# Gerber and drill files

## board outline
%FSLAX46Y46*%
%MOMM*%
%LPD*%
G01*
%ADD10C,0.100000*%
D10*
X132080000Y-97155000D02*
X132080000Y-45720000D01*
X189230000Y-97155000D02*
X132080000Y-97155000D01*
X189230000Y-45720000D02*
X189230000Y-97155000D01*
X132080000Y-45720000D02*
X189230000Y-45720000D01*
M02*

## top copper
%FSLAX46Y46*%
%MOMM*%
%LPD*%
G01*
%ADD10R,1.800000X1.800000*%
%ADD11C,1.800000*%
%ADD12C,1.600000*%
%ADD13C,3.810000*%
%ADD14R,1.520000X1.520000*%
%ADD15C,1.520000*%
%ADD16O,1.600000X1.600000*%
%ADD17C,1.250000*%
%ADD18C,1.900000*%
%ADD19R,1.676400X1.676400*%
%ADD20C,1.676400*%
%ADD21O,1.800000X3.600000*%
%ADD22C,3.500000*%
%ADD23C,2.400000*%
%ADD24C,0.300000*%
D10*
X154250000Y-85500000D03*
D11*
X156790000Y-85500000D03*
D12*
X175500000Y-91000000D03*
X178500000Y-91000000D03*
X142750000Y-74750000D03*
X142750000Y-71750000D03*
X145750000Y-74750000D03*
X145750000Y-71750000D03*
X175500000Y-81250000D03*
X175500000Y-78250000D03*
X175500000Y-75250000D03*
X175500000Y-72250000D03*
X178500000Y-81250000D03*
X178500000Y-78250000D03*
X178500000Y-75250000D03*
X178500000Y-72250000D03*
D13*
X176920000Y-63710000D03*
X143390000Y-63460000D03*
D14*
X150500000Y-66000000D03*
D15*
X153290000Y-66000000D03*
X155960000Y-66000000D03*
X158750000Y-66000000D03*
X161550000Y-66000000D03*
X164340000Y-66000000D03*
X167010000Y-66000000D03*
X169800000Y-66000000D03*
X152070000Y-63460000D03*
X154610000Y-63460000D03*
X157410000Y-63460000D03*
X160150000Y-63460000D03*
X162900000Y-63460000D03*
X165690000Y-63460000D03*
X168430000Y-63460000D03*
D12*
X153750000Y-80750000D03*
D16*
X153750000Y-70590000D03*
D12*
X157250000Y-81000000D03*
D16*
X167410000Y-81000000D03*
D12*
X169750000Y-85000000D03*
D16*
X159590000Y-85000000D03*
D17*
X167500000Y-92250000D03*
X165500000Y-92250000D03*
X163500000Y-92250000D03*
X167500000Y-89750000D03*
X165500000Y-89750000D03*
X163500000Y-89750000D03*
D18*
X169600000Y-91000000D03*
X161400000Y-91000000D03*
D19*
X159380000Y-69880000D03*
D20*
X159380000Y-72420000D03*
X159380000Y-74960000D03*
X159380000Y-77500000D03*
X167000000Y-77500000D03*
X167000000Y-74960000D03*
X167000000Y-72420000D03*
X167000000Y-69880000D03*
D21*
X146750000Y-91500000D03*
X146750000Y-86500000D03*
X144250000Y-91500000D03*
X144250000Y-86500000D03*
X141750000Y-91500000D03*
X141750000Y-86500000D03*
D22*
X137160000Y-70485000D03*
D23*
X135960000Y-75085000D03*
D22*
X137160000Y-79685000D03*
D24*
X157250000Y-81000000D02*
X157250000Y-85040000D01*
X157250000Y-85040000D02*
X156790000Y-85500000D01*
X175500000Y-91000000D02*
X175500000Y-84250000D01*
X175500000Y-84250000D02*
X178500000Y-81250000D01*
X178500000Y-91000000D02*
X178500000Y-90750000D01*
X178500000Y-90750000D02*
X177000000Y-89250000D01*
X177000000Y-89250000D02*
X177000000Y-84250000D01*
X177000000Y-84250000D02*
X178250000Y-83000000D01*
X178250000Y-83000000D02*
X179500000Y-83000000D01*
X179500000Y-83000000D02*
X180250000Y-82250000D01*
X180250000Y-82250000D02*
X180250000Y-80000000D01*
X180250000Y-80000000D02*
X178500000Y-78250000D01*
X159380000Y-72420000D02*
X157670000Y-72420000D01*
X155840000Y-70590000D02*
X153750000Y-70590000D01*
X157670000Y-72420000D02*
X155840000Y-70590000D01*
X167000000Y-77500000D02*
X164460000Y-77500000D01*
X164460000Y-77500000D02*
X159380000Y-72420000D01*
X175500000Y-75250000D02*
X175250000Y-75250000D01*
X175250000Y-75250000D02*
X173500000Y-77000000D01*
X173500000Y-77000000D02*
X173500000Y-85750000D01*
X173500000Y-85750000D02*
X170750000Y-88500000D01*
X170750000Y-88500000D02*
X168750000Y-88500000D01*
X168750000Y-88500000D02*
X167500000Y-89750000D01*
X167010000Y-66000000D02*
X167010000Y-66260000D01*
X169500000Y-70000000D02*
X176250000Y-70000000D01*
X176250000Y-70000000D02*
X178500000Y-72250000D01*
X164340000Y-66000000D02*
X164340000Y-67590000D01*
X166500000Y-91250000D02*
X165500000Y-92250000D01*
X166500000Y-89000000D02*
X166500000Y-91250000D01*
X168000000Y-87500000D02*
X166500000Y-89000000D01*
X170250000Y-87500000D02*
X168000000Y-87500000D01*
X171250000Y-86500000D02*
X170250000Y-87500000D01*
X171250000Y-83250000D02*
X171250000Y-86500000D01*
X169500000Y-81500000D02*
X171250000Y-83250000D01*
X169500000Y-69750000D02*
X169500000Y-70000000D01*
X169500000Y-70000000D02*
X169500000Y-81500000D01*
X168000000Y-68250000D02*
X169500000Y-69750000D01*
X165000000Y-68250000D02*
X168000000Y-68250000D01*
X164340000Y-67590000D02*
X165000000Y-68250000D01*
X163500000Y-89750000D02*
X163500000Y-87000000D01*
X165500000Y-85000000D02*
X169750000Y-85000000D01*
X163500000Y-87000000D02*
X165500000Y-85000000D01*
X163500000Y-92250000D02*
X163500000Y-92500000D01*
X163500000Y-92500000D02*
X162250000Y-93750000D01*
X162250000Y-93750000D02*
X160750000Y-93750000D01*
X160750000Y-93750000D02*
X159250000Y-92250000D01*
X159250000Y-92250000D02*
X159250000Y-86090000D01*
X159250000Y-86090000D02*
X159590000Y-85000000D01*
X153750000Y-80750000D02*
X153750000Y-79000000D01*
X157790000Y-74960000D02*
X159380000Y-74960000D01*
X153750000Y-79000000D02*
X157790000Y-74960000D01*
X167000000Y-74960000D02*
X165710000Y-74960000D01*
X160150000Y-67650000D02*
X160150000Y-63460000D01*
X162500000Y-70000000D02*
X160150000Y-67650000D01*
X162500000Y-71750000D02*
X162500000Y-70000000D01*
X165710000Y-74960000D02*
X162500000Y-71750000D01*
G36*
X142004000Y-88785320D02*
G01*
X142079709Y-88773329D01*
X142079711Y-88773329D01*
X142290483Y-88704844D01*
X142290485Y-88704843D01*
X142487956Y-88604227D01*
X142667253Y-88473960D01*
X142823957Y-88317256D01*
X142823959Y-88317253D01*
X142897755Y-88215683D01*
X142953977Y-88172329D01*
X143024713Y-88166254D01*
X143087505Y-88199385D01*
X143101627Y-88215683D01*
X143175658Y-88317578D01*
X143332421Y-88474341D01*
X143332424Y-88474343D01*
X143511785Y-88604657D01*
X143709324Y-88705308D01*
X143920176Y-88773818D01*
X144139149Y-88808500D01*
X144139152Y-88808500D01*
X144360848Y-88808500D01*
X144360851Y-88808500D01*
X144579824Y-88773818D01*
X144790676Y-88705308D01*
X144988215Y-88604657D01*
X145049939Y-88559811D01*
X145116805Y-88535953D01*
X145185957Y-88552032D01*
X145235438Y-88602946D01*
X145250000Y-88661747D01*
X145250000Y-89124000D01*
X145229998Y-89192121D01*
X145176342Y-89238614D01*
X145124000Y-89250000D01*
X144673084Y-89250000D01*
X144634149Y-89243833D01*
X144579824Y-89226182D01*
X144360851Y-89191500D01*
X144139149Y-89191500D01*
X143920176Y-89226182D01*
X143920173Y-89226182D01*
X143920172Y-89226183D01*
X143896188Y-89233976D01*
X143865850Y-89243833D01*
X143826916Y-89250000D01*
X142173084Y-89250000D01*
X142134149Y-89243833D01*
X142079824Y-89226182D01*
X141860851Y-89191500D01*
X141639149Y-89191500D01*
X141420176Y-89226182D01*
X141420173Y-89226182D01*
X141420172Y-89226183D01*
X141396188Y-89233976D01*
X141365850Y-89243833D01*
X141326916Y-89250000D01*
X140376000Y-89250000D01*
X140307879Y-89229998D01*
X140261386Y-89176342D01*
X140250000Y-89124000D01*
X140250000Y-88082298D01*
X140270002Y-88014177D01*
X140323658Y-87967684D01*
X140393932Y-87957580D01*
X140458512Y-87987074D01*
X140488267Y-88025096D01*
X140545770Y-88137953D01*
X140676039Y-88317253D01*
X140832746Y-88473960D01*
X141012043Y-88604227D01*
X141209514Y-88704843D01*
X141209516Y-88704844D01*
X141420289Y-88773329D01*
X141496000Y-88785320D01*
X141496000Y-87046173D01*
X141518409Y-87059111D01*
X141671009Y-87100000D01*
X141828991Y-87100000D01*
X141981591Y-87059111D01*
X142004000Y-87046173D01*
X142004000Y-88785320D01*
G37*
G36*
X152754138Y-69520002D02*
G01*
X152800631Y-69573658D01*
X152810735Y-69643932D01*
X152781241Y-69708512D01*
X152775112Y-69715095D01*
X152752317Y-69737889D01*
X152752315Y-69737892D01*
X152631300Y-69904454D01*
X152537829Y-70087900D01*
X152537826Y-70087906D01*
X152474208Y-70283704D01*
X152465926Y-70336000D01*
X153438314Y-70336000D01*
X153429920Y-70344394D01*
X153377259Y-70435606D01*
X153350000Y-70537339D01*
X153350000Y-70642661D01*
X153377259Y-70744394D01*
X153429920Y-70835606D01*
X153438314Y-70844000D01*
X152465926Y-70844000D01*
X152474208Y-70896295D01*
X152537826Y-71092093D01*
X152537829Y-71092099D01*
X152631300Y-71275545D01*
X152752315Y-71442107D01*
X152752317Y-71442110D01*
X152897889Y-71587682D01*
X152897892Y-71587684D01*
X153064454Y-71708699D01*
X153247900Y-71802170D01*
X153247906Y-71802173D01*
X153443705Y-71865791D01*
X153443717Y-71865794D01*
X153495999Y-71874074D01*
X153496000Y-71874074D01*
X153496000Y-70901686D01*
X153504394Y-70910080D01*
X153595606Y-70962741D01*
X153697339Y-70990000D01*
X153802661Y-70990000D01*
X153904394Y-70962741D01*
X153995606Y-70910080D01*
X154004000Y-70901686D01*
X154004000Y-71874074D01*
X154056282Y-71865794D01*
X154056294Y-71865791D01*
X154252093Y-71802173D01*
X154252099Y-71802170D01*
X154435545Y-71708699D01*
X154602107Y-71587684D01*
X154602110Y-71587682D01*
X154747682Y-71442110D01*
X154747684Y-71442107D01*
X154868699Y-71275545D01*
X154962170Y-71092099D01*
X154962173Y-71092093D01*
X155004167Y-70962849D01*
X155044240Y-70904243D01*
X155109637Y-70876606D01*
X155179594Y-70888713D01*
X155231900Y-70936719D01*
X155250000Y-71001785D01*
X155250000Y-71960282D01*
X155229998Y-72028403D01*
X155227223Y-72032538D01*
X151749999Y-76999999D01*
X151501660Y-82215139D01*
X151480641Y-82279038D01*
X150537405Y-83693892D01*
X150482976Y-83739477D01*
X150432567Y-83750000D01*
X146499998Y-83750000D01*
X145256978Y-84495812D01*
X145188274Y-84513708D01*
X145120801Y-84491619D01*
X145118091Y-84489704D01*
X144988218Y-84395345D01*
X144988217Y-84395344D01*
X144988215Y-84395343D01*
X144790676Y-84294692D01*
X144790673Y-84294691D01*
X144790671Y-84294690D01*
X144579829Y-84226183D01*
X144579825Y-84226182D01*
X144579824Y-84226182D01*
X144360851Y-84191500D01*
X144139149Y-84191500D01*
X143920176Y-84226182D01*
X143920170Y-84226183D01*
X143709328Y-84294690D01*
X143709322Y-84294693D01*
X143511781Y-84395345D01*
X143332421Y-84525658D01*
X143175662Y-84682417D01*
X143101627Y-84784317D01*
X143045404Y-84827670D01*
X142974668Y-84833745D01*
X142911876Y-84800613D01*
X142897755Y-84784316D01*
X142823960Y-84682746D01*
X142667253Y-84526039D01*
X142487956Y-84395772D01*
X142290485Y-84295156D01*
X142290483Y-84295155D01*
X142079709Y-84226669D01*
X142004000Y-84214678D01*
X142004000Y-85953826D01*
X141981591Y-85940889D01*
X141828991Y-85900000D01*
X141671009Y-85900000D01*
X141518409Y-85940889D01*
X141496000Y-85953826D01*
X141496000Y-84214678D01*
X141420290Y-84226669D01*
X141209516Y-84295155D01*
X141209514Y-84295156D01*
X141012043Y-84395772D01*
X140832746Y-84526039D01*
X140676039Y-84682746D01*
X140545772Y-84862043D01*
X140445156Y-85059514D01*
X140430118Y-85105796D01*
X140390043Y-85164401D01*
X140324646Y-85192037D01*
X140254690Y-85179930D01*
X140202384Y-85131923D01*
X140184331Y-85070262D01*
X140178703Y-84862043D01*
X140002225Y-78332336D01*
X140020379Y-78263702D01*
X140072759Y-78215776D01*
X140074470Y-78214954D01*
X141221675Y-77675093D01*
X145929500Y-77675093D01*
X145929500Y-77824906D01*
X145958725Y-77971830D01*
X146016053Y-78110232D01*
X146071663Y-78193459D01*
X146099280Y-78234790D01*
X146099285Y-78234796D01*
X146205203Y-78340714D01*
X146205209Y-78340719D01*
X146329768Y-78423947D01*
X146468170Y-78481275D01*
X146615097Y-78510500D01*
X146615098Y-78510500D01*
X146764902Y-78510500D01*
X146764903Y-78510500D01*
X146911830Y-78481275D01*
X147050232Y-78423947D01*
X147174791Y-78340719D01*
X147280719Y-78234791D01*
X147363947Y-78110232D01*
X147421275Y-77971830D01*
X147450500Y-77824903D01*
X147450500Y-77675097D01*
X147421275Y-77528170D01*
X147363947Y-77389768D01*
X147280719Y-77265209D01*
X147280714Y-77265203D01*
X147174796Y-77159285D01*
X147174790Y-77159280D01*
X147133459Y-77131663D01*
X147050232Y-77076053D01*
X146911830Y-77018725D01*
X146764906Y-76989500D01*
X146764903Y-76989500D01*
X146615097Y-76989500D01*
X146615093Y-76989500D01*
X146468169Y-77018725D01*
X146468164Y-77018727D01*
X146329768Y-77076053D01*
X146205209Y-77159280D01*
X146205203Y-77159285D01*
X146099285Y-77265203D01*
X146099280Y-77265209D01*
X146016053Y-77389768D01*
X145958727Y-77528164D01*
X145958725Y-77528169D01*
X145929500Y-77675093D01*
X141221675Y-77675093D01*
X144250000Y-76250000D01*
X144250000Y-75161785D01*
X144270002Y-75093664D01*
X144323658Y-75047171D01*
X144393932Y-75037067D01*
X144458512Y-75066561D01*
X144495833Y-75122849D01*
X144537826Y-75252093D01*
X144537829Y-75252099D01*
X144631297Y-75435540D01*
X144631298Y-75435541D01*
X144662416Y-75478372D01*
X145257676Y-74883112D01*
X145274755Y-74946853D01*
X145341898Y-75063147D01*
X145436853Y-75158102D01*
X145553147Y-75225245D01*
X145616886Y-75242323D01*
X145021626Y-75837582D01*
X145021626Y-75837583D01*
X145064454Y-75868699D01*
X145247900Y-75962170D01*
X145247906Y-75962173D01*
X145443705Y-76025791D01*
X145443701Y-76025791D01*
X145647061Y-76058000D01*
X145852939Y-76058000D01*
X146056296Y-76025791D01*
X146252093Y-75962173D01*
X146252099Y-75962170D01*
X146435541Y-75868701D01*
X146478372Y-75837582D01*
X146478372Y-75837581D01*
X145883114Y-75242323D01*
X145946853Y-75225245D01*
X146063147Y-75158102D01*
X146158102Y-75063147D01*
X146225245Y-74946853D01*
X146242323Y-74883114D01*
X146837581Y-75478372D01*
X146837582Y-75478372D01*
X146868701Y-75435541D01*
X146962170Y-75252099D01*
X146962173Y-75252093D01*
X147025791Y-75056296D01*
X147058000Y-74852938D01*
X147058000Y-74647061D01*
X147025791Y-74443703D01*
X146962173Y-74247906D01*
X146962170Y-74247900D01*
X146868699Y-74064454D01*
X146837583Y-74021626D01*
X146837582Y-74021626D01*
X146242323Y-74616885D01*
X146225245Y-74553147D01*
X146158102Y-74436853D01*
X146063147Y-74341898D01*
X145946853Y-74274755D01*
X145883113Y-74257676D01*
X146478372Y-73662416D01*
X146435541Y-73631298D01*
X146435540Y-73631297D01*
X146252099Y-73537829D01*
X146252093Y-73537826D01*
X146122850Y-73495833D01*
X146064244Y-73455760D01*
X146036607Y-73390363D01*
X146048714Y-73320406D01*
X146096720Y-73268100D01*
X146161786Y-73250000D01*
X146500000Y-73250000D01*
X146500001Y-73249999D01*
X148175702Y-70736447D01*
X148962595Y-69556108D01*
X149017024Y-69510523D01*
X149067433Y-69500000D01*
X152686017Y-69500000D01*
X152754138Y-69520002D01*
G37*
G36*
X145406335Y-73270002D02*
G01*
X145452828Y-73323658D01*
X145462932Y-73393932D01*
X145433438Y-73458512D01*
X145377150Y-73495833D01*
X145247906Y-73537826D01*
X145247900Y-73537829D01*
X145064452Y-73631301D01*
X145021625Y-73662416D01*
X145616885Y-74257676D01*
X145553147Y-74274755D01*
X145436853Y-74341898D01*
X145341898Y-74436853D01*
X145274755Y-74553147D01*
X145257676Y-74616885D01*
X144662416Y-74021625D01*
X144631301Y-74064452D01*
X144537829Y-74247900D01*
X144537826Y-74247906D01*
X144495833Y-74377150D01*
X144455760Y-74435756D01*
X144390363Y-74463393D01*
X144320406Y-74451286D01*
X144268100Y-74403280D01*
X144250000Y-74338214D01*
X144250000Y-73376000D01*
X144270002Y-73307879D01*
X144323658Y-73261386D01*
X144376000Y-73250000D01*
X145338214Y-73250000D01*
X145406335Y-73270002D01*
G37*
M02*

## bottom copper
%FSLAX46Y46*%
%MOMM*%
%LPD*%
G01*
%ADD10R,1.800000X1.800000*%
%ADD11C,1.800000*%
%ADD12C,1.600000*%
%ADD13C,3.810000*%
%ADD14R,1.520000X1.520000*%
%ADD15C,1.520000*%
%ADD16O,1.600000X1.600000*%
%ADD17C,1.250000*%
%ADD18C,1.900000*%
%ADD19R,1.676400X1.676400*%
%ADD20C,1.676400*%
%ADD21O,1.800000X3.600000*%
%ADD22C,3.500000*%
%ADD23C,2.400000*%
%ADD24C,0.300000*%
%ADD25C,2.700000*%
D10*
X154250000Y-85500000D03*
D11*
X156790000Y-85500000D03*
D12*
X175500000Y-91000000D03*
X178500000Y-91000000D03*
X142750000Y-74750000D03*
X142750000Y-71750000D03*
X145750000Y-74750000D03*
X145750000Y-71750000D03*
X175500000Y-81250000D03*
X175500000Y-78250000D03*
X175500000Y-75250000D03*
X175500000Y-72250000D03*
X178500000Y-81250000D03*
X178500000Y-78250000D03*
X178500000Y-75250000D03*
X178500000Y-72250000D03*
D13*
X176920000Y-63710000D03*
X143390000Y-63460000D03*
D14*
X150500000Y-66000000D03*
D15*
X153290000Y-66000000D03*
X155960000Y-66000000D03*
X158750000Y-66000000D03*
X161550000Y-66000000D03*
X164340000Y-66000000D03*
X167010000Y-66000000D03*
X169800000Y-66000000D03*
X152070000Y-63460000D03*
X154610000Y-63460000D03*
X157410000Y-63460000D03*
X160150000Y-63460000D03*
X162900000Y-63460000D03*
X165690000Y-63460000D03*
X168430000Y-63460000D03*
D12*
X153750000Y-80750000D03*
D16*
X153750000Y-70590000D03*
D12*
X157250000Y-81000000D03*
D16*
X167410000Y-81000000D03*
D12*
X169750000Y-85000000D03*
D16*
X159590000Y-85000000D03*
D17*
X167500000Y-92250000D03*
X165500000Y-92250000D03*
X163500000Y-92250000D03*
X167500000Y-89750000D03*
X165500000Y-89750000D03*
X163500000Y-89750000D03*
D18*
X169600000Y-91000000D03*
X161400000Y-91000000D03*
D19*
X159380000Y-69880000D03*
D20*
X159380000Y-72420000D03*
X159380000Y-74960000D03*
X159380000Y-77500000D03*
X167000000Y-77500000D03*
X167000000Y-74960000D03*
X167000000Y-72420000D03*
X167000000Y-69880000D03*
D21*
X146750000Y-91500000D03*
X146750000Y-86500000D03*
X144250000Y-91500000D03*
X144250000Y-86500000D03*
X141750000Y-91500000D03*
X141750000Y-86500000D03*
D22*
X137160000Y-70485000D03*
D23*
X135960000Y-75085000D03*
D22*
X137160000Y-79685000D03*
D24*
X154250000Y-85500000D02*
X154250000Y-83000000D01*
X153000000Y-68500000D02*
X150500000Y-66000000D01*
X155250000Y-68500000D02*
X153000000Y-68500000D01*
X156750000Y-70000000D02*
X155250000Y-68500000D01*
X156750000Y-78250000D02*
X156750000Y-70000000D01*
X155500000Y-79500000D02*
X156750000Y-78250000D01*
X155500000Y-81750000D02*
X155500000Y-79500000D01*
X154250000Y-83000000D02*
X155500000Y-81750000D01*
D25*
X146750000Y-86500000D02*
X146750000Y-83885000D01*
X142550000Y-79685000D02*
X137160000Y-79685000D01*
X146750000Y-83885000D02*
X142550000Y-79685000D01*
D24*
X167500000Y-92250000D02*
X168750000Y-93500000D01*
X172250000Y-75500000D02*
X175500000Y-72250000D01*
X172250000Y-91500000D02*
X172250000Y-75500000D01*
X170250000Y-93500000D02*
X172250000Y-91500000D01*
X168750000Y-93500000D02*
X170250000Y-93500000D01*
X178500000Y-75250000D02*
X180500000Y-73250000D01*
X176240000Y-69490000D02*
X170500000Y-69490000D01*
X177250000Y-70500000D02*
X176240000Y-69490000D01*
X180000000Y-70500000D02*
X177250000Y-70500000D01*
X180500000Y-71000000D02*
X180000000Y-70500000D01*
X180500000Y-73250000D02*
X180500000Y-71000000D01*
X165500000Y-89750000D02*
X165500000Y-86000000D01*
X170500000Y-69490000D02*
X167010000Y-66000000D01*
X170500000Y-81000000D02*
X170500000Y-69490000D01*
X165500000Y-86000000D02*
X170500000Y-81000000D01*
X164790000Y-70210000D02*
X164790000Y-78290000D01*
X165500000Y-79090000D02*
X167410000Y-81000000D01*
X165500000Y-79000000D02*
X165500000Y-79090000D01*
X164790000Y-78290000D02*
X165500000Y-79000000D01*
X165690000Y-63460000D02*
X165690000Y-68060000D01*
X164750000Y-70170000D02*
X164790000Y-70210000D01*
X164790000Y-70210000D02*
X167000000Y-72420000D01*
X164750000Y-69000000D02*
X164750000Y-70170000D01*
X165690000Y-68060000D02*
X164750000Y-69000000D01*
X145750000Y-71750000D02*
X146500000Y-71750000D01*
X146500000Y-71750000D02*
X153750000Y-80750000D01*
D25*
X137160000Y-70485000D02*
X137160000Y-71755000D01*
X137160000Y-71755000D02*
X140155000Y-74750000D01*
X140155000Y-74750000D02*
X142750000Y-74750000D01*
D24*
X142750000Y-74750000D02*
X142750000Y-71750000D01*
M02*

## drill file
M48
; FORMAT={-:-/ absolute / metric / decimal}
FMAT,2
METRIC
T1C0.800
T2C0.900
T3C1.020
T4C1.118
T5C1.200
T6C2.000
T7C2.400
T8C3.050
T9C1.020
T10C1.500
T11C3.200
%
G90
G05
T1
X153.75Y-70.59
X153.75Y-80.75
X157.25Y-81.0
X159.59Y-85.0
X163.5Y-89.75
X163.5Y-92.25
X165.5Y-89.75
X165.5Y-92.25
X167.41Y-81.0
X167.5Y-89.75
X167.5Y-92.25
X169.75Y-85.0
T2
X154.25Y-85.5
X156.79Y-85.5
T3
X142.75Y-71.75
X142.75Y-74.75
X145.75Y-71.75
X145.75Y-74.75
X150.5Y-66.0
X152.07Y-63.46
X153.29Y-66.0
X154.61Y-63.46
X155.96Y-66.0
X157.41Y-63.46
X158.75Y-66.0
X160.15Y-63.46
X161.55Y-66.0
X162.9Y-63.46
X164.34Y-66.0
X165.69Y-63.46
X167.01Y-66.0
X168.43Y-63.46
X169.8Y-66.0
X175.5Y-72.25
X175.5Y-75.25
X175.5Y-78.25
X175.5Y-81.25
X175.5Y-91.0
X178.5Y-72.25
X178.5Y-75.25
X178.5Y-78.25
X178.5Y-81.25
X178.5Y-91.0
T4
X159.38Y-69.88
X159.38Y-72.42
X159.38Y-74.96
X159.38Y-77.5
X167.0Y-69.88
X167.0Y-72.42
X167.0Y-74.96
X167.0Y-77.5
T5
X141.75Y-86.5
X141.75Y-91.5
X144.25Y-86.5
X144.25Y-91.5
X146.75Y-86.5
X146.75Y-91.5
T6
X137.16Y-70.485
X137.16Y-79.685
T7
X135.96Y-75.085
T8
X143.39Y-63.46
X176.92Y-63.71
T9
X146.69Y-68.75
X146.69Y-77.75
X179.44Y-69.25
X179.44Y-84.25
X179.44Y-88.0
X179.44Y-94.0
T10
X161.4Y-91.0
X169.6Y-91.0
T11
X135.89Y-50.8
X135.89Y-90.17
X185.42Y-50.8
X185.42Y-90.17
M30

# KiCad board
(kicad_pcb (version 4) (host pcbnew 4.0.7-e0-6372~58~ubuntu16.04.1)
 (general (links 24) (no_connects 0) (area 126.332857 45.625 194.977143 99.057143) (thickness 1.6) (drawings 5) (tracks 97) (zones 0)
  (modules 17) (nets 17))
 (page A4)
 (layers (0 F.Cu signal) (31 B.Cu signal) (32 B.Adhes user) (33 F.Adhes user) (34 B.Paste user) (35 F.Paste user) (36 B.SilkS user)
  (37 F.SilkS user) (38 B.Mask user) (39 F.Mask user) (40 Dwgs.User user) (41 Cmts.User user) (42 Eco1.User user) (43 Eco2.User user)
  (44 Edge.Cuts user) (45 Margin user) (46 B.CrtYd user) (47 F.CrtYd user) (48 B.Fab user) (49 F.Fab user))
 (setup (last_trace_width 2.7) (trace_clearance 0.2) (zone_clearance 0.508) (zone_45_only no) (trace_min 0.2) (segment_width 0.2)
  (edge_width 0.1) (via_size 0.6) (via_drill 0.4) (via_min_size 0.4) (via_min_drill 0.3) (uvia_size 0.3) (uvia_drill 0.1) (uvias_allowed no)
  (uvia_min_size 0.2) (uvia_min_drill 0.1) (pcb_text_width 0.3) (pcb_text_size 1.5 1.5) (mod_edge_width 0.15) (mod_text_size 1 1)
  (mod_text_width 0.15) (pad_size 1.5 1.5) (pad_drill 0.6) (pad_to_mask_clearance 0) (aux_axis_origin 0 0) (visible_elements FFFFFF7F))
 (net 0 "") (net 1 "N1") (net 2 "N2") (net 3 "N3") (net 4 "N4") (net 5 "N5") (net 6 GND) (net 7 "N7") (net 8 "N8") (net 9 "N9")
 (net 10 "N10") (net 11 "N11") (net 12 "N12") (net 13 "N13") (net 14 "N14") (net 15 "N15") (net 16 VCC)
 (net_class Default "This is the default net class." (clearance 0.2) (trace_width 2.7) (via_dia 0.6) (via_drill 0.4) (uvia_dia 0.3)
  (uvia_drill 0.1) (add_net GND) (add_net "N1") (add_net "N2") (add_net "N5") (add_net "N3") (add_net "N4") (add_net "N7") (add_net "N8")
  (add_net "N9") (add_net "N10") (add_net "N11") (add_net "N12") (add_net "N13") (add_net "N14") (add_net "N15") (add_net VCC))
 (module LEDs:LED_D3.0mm (layer F.Cu) (at 154.25 85.5)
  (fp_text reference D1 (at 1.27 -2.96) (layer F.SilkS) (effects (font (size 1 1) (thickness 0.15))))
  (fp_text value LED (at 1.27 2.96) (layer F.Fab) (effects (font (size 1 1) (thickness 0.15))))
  (pad 1 thru_hole rect (at 0 0) (size 1.8 1.8) (drill 0.9) (layers *.Cu *.Mask) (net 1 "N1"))
  (pad 2 thru_hole circle (at 2.54 0) (size 1.8 1.8) (drill 0.9) (layers *.Cu *.Mask) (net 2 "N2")))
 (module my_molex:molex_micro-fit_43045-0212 (layer F.Cu) (at 178.5 91 270)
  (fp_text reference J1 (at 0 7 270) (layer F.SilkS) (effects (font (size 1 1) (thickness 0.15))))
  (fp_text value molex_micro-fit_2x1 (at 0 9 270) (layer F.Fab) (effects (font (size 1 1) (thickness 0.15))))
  (pad 1 thru_hole circle (at 0 3 270) (size 1.6 1.6) (drill 1.02) (layers *.Cu *.Mask) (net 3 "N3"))
  (pad 2 thru_hole circle (at 0 0 270) (size 1.6 1.6) (drill 1.02) (layers *.Cu *.Mask) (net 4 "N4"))
  (pad "" np_thru_hole circle (at -3 -0.94 270) (size 1.02 1.02) (drill 1.02) (layers *.Cu *.Mask))
  (pad "" np_thru_hole circle (at 3 -0.94 270) (size 1.02 1.02) (drill 1.02) (layers *.Cu *.Mask)))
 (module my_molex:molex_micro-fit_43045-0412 (layer F.Cu) (at 145.75 73.25 270)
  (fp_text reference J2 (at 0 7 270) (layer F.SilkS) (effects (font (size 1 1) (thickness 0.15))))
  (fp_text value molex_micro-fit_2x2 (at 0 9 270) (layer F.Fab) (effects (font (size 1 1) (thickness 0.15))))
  (pad 1 thru_hole circle (at 1.5 3 270) (size 1.6 1.6) (drill 1.02) (layers *.Cu *.Mask) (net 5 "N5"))
  (pad 2 thru_hole circle (at -1.5 3 270) (size 1.6 1.6) (drill 1.02) (layers *.Cu *.Mask) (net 5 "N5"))
  (pad 3 thru_hole circle (at 1.5 0 270) (size 1.6 1.6) (drill 1.02) (layers *.Cu *.Mask) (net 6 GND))
  (pad 4 thru_hole circle (at -1.5 0 270) (size 1.6 1.6) (drill 1.02) (layers *.Cu *.Mask) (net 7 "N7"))
  (pad "" np_thru_hole circle (at -4.5 -0.94 270) (size 1.02 1.02) (drill 1.02) (layers *.Cu *.Mask))
  (pad "" np_thru_hole circle (at 4.5 -0.94 270) (size 1.02 1.02) (drill 1.02) (layers *.Cu *.Mask)))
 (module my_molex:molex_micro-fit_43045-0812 (layer F.Cu) (at 178.5 76.75 270)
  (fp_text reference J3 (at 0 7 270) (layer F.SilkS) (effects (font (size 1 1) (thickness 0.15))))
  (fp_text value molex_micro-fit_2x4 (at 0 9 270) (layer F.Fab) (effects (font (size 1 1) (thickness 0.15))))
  (pad 1 thru_hole circle (at 4.5 3 270) (size 1.6 1.6) (drill 1.02) (layers *.Cu *.Mask))
  (pad 2 thru_hole circle (at 1.5 3 270) (size 1.6 1.6) (drill 1.02) (layers *.Cu *.Mask))
  (pad 3 thru_hole circle (at -1.5 3 270) (size 1.6 1.6) (drill 1.02) (layers *.Cu *.Mask) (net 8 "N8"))
  (pad 4 thru_hole circle (at -4.5 3 270) (size 1.6 1.6) (drill 1.02) (layers *.Cu *.Mask) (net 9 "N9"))
  (pad 5 thru_hole circle (at 4.5 0 270) (size 1.6 1.6) (drill 1.02) (layers *.Cu *.Mask) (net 3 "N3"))
  (pad 6 thru_hole circle (at 1.5 0 270) (size 1.6 1.6) (drill 1.02) (layers *.Cu *.Mask) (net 4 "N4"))
  (pad 7 thru_hole circle (at -1.5 0 270) (size 1.6 1.6) (drill 1.02) (layers *.Cu *.Mask) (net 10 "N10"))
  (pad 8 thru_hole circle (at -4.5 0 270) (size 1.6 1.6) (drill 1.02) (layers *.Cu *.Mask) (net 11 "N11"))
  (pad "" np_thru_hole circle (at -7.5 -0.94 270) (size 1.02 1.02) (drill 1.02) (layers *.Cu *.Mask))
  (pad "" np_thru_hole circle (at 7.5 -0.94 270) (size 1.02 1.02) (drill 1.02) (layers *.Cu *.Mask)))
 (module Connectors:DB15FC (layer F.Cu) (at 150.5 66)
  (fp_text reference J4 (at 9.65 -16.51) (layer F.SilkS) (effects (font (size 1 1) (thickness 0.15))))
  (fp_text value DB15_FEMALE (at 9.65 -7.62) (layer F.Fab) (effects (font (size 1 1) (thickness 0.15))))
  (pad "" thru_hole circle (at 26.42 -2.29) (size 3.81 3.81) (drill 3.05) (layers *.Cu *.Mask))
  (pad "" thru_hole circle (at -7.11 -2.54) (size 3.81 3.81) (drill 3.05) (layers *.Cu *.Mask))
  (pad 1 thru_hole rect (at 0 0) (size 1.52 1.52) (drill 1.02) (layers *.Cu *.Mask) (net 1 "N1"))
  (pad 2 thru_hole circle (at 2.79 0) (size 1.52 1.52) (drill 1.02) (layers *.Cu *.Mask))
  (pad 3 thru_hole circle (at 5.46 0) (size 1.52 1.52) (drill 1.02) (layers *.Cu *.Mask))
  (pad 4 thru_hole circle (at 8.25 0) (size 1.52 1.52) (drill 1.02) (layers *.Cu *.Mask))
  (pad 5 thru_hole circle (at 11.05 0) (size 1.52 1.52) (drill 1.02) (layers *.Cu *.Mask))
  (pad 6 thru_hole circle (at 13.84 0) (size 1.52 1.52) (drill 1.02) (layers *.Cu *.Mask) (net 11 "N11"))
  (pad 7 thru_hole circle (at 16.51 0) (size 1.52 1.52) (drill 1.02) (layers *.Cu *.Mask) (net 10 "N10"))
  (pad 8 thru_hole circle (at 19.3 0) (size 1.52 1.52) (drill 1.02) (layers *.Cu *.Mask))
  (pad 9 thru_hole circle (at 1.57 -2.54) (size 1.52 1.52) (drill 1.02) (layers *.Cu *.Mask))
  (pad 10 thru_hole circle (at 4.11 -2.54) (size 1.52 1.52) (drill 1.02) (layers *.Cu *.Mask))
  (pad 11 thru_hole circle (at 6.91 -2.54) (size 1.52 1.52) (drill 1.02) (layers *.Cu *.Mask))
  (pad 12 thru_hole circle (at 9.65 -2.54) (size 1.52 1.52) (drill 1.02) (layers *.Cu *.Mask) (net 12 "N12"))
  (pad 13 thru_hole circle (at 12.4 -2.54) (size 1.52 1.52) (drill 1.02) (layers *.Cu *.Mask))
  (pad 14 thru_hole circle (at 15.19 -2.54) (size 1.52 1.52) (drill 1.02) (layers *.Cu *.Mask) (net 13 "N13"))
  (pad 15 thru_hole circle (at 17.93 -2.54) (size 1.52 1.52) (drill 1.02) (layers *.Cu *.Mask)))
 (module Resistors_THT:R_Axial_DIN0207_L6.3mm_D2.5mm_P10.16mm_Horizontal (layer F.Cu) (at 153.75 80.75 90)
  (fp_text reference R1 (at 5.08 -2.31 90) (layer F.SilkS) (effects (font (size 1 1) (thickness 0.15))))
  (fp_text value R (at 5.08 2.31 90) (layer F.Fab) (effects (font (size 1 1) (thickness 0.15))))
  (pad 1 thru_hole circle (at 0 0 90) (size 1.6 1.6) (drill 0.8) (layers *.Cu *.Mask) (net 7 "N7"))
  (pad 2 thru_hole oval (at 10.16 0 90) (size 1.6 1.6) (drill 0.8) (layers *.Cu *.Mask) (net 6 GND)))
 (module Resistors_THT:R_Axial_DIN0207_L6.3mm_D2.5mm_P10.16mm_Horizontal (layer F.Cu) (at 157.25 81)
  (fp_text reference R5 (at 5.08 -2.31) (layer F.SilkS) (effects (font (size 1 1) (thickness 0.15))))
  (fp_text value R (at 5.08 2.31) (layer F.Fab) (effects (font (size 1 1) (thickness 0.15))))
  (pad 1 thru_hole circle (at 0 0) (size 1.6 1.6) (drill 0.8) (layers *.Cu *.Mask) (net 2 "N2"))
  (pad 2 thru_hole oval (at 10.16 0) (size 1.6 1.6) (drill 0.8) (layers *.Cu *.Mask) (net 13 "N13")))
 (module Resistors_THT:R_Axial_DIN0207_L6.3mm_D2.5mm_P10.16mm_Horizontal (layer F.Cu) (at 169.75 85 180)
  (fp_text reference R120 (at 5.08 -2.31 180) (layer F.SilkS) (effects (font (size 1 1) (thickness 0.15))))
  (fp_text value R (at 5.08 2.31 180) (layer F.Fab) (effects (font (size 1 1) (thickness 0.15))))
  (pad 1 thru_hole circle (at 0 0 180) (size 1.6 1.6) (drill 0.8) (layers *.Cu *.Mask) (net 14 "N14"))
  (pad 2 thru_hole oval (at 10.16 0 180) (size 1.6 1.6) (drill 0.8) (layers *.Cu *.Mask) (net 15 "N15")))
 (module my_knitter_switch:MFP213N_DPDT (layer F.Cu) (at 165.5 91 180)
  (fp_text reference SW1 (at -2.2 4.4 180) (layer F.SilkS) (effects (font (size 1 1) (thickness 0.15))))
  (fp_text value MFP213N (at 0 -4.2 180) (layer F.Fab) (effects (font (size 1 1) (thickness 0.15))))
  (pad 1 thru_hole circle (at -2 -1.25 180) (size 1.25 1.25) (drill 0.8) (layers *.Cu *.Mask) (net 9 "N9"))
  (pad 2 thru_hole circle (at 0 -1.25 180) (size 1.25 1.25) (drill 0.8) (layers *.Cu *.Mask) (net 11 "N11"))
  (pad 3 thru_hole circle (at 2 -1.25 180) (size 1.25 1.25) (drill 0.8) (layers *.Cu *.Mask) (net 15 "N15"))
  (pad 4 thru_hole circle (at -2 1.25 180) (size 1.25 1.25) (drill 0.8) (layers *.Cu *.Mask) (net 8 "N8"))
  (pad 5 thru_hole circle (at 0 1.25 180) (size 1.25 1.25) (drill 0.8) (layers *.Cu *.Mask) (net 10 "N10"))
  (pad 6 thru_hole circle (at 2 1.25 180) (size 1.25 1.25) (drill 0.8) (layers *.Cu *.Mask) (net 14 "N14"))
  (pad "" np_thru_hole circle (at -4.1 0 180) (size 1.9 1.9) (drill 1.5) (layers *.Cu *.Mask))
  (pad "" np_thru_hole circle (at 4.1 0 180) (size 1.9 1.9) (drill 1.5) (layers *.Cu *.Mask)))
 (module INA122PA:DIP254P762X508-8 (layer F.Cu) (at 167 77.5)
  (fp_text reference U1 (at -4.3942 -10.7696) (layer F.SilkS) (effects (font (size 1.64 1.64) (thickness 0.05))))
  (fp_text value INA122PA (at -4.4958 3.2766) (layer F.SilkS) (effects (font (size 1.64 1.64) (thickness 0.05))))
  (pad 1 thru_hole rect (at -7.62 -7.62) (size 1.6764 1.6764) (drill 1.1176) (layers *.Cu *.Mask F.SilkS))
  (pad 2 thru_hole circle (at -7.62 -5.08) (size 1.6764 1.6764) (drill 1.1176) (layers *.Cu *.Mask F.SilkS) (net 6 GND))
  (pad 3 thru_hole circle (at -7.62 -2.54) (size 1.6764 1.6764) (drill 1.1176) (layers *.Cu *.Mask F.SilkS) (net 7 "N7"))
  (pad 4 thru_hole circle (at -7.62 0) (size 1.6764 1.6764) (drill 1.1176) (layers *.Cu *.Mask F.SilkS))
  (pad 5 thru_hole circle (at 0 0) (size 1.6764 1.6764) (drill 1.1176) (layers *.Cu *.Mask F.SilkS) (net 6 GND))
  (pad 6 thru_hole circle (at 0 -2.54) (size 1.6764 1.6764) (drill 1.1176) (layers *.Cu *.Mask F.SilkS) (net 12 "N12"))
  (pad 7 thru_hole circle (at 0 -5.08) (size 1.6764 1.6764) (drill 1.1176) (layers *.Cu *.Mask F.SilkS) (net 13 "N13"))
  (pad 8 thru_hole circle (at 0 -7.62) (size 1.6764 1.6764) (drill 1.1176) (layers *.Cu *.Mask F.SilkS)))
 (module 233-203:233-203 (layer F.Cu) (at 144.25 89 180)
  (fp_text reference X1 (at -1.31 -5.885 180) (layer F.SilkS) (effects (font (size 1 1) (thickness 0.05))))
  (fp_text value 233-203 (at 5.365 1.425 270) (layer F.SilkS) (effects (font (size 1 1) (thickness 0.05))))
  (pad A1 thru_hole oval (at -2.5 -2.5 270) (size 3.6 1.8) (drill 1.2) (layers *.Cu *.Mask F.SilkS))
  (pad B1 thru_hole oval (at -2.5 2.5 270) (size 3.6 1.8) (drill 1.2) (layers *.Cu *.Mask F.SilkS) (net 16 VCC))
  (pad A2 thru_hole oval (at 0 -2.5 270) (size 3.6 1.8) (drill 1.2) (layers *.Cu *.Mask F.SilkS))
  (pad B2 thru_hole oval (at 0 2.5 270) (size 3.6 1.8) (drill 1.2) (layers *.Cu *.Mask F.SilkS))
  (pad A3 thru_hole oval (at 2.5 -2.5 270) (size 3.6 1.8) (drill 1.2) (layers *.Cu *.Mask F.SilkS))
  (pad B3 thru_hole oval (at 2.5 2.5 270) (size 3.6 1.8) (drill 1.2) (layers *.Cu *.Mask F.SilkS) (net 6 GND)))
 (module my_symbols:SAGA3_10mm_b (layer F.Cu) (at 156.5 92.5)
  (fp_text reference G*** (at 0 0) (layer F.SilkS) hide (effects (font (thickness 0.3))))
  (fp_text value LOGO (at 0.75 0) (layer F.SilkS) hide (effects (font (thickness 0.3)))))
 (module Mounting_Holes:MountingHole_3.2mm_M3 (layer F.Cu) (at 185.42 50.8)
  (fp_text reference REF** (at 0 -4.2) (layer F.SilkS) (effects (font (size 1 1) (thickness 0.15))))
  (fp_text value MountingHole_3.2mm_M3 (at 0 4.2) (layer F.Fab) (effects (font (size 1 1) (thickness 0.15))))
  (pad 1 np_thru_hole circle (at 0 0) (size 3.2 3.2) (drill 3.2) (layers *.Cu *.Mask)))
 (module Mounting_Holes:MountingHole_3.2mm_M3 (layer F.Cu) (at 135.89 50.8)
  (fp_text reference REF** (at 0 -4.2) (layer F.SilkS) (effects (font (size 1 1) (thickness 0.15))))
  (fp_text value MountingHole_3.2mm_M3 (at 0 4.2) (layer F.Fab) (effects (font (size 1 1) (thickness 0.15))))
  (pad 1 np_thru_hole circle (at 0 0) (size 3.2 3.2) (drill 3.2) (layers *.Cu *.Mask)))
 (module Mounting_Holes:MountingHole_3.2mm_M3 (layer F.Cu) (at 135.89 90.17)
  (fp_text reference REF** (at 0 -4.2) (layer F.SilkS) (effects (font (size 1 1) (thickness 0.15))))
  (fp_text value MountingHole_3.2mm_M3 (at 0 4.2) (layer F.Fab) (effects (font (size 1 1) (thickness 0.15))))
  (pad 1 np_thru_hole circle (at 0 0) (size 3.2 3.2) (drill 3.2) (layers *.Cu *.Mask)))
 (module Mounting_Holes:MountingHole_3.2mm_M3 (layer F.Cu) (at 185.42 90.17)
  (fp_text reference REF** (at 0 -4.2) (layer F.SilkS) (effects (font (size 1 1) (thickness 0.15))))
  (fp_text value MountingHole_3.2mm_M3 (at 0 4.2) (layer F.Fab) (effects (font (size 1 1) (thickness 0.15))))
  (pad 1 np_thru_hole circle (at 0 0) (size 3.2 3.2) (drill 3.2) (layers *.Cu *.Mask)))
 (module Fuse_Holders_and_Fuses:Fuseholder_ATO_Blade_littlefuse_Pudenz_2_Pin (layer F.Cu) (at 137.16 70.485 270)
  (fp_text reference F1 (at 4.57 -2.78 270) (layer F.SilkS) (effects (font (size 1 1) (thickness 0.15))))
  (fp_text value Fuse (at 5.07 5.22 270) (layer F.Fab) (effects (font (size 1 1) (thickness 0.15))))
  (pad 1 thru_hole circle (at 0 0 270) (size 3.5 3.5) (drill 2) (layers *.Cu *.Mask) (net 5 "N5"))
  (pad "" thru_hole circle (at 4.6 1.2 270) (size 2.4 2.4) (drill 2.4) (layers *.Cu *.Mask))
  (pad 2 thru_hole circle (at 9.2 0 270) (size 3.5 3.5) (drill 2) (layers *.Cu *.Mask) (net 16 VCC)))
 (gr_line (start 132.08 97.155) (end 132.08 45.72) (angle 90) (layer Edge.Cuts) (width 0.1))
 (gr_line (start 189.23 97.155) (end 132.08 97.155) (angle 90) (layer Edge.Cuts) (width 0.1))
 (gr_line (start 189.23 45.72) (end 189.23 97.155) (angle 90) (layer Edge.Cuts) (width 0.1))
 (gr_line (start 132.08 45.72) (end 189.23 45.72) (angle 90) (layer Edge.Cuts) (width 0.1))
 (segment (start 154.25 85.5) (end 154.25 83) (width 0.3) (layer B.Cu) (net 1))
 (segment (start 153 68.5) (end 150.5 66) (width 0.3) (layer B.Cu) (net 1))
 (segment (start 155.25 68.5) (end 153 68.5) (width 0.3) (layer B.Cu) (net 1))
 (segment (start 156.75 70) (end 155.25 68.5) (width 0.3) (layer B.Cu) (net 1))
 (segment (start 156.75 78.25) (end 156.75 70) (width 0.3) (layer B.Cu) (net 1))
 (segment (start 155.5 79.5) (end 156.75 78.25) (width 0.3) (layer B.Cu) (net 1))
 (segment (start 155.5 81.75) (end 155.5 79.5) (width 0.3) (layer B.Cu) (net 1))
 (segment (start 154.25 83) (end 155.5 81.75) (width 0.3) (layer B.Cu) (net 1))
 (segment (start 157.25 81) (end 157.25 85.04) (width 0.3) (layer F.Cu) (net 2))
 (segment (start 157.25 85.04) (end 156.79 85.5) (width 0.3) (layer F.Cu) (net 2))
 (segment (start 175.5 91) (end 175.5 84.25) (width 0.3) (layer F.Cu) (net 3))
 (segment (start 175.5 84.25) (end 178.5 81.25) (width 0.3) (layer F.Cu) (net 3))
 (segment (start 178.5 91) (end 178.5 90.75) (width 0.3) (layer F.Cu) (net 4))
 (segment (start 178.5 90.75) (end 177 89.25) (width 0.3) (layer F.Cu) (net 4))
 (segment (start 177 89.25) (end 177 84.25) (width 0.3) (layer F.Cu) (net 4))
 (segment (start 177 84.25) (end 178.25 83) (width 0.3) (layer F.Cu) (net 4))
 (segment (start 178.25 83) (end 179.5 83) (width 0.3) (layer F.Cu) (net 4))
 (segment (start 179.5 83) (end 180.25 82.25) (width 0.3) (layer F.Cu) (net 4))
 (segment (start 180.25 82.25) (end 180.25 80) (width 0.3) (layer F.Cu) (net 4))
 (segment (start 180.25 80) (end 178.5 78.25) (width 0.3) (layer F.Cu) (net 4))
 (segment (start 159.38 72.42) (end 157.67 72.42) (width 0.3) (layer F.Cu) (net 6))
 (segment (start 155.84 70.59) (end 153.75 70.59) (width 0.3) (layer F.Cu) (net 6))
 (segment (start 157.67 72.42) (end 155.84 70.59) (width 0.3) (layer F.Cu) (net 6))
 (segment (start 167 77.5) (end 164.46 77.5) (width 0.3) (layer F.Cu) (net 6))
 (segment (start 164.46 77.5) (end 159.38 72.42) (width 0.3) (layer F.Cu) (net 6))
 (segment (start 146.75 86.5) (end 146.75 83.885) (width 2.7) (layer B.Cu) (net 16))
 (segment (start 142.55 79.685) (end 137.16 79.685) (width 2.7) (layer B.Cu) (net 16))
 (segment (start 146.75 83.885) (end 142.55 79.685) (width 2.7) (layer B.Cu) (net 16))
 (segment (start 175.5 75.25) (end 175.25 75.25) (width 0.3) (layer F.Cu) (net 8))
 (segment (start 175.25 75.25) (end 173.5 77) (width 0.3) (layer F.Cu) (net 8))
 (segment (start 173.5 77) (end 173.5 85.75) (width 0.3) (layer F.Cu) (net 8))
 (segment (start 173.5 85.75) (end 170.75 88.5) (width 0.3) (layer F.Cu) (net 8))
 (segment (start 170.75 88.5) (end 168.75 88.5) (width 0.3) (layer F.Cu) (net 8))
 (segment (start 168.75 88.5) (end 167.5 89.75) (width 0.3) (layer F.Cu) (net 8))
 (segment (start 167.5 92.25) (end 168.75 93.5) (width 0.3) (layer B.Cu) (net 9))
 (segment (start 172.25 75.5) (end 175.5 72.25) (width 0.3) (layer B.Cu) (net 9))
 (segment (start 172.25 91.5) (end 172.25 75.5) (width 0.3) (layer B.Cu) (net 9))
 (segment (start 170.25 93.5) (end 172.25 91.5) (width 0.3) (layer B.Cu) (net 9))
 (segment (start 168.75 93.5) (end 170.25 93.5) (width 0.3) (layer B.Cu) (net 9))
 (segment (start 178.5 75.25) (end 180.5 73.25) (width 0.3) (layer B.Cu) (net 10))
 (segment (start 176.24 69.49) (end 170.5 69.49) (width 0.3) (layer B.Cu) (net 10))
 (segment (start 177.25 70.5) (end 176.24 69.49) (width 0.3) (layer B.Cu) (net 10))
 (segment (start 180 70.5) (end 177.25 70.5) (width 0.3) (layer B.Cu) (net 10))
 (segment (start 180.5 71) (end 180 70.5) (width 0.3) (layer B.Cu) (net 10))
 (segment (start 180.5 73.25) (end 180.5 71) (width 0.3) (layer B.Cu) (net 10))
 (segment (start 165.5 89.75) (end 165.5 86) (width 0.3) (layer B.Cu) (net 10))
 (segment (start 170.5 69.49) (end 167.01 66) (width 0.3) (layer B.Cu) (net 10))
 (segment (start 170.5 81) (end 170.5 69.49) (width 0.3) (layer B.Cu) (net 10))
 (segment (start 165.5 86) (end 170.5 81) (width 0.3) (layer B.Cu) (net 10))
 (segment (start 167.01 66) (end 167.01 66.26) (width 0.3) (layer F.Cu) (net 10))
 (segment (start 169.5 70) (end 176.25 70) (width 0.3) (layer F.Cu) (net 11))
 (segment (start 176.25 70) (end 178.5 72.25) (width 0.3) (layer F.Cu) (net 11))
 (segment (start 164.34 66) (end 164.34 67.59) (width 0.3) (layer F.Cu) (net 11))
 (segment (start 166.5 91.25) (end 165.5 92.25) (width 0.3) (layer F.Cu) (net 11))
 (segment (start 166.5 89) (end 166.5 91.25) (width 0.3) (layer F.Cu) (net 11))
 (segment (start 168 87.5) (end 166.5 89) (width 0.3) (layer F.Cu) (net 11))
 (segment (start 170.25 87.5) (end 168 87.5) (width 0.3) (layer F.Cu) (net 11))
 (segment (start 171.25 86.5) (end 170.25 87.5) (width 0.3) (layer F.Cu) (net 11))
 (segment (start 171.25 83.25) (end 171.25 86.5) (width 0.3) (layer F.Cu) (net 11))
 (segment (start 169.5 81.5) (end 171.25 83.25) (width 0.3) (layer F.Cu) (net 11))
 (segment (start 169.5 69.75) (end 169.5 70) (width 0.3) (layer F.Cu) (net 11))
 (segment (start 169.5 70) (end 169.5 81.5) (width 0.3) (layer F.Cu) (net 11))
 (segment (start 168 68.25) (end 169.5 69.75) (width 0.3) (layer F.Cu) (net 11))
 (segment (start 165 68.25) (end 168 68.25) (width 0.3) (layer F.Cu) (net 11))
 (segment (start 164.34 67.59) (end 165 68.25) (width 0.3) (layer F.Cu) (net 11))
 (segment (start 164.79 70.21) (end 164.79 78.29) (width 0.3) (layer B.Cu) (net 13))
 (segment (start 165.5 79.09) (end 167.41 81) (width 0.3) (layer B.Cu) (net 13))
 (segment (start 165.5 79) (end 165.5 79.09) (width 0.3) (layer B.Cu) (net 13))
 (segment (start 164.79 78.29) (end 165.5 79) (width 0.3) (layer B.Cu) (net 13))
 (segment (start 165.69 63.46) (end 165.69 68.06) (width 0.3) (layer B.Cu) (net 13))
 (segment (start 164.75 70.17) (end 164.79 70.21) (width 0.3) (layer B.Cu) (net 13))
 (segment (start 164.79 70.21) (end 167 72.42) (width 0.3) (layer B.Cu) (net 13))
 (segment (start 164.75 69) (end 164.75 70.17) (width 0.3) (layer B.Cu) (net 13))
 (segment (start 165.69 68.06) (end 164.75 69) (width 0.3) (layer B.Cu) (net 13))
 (segment (start 163.5 89.75) (end 163.5 87) (width 0.3) (layer F.Cu) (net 14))
 (segment (start 165.5 85) (end 169.75 85) (width 0.3) (layer F.Cu) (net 14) (status 20))
 (segment (start 163.5 87) (end 165.5 85) (width 0.3) (layer F.Cu) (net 14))
 (segment (start 163.5 92.25) (end 163.5 92.5) (width 0.3) (layer F.Cu) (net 15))
 (segment (start 163.5 92.5) (end 162.25 93.75) (width 0.3) (layer F.Cu) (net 15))
 (segment (start 162.25 93.75) (end 160.75 93.75) (width 0.3) (layer F.Cu) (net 15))
 (segment (start 160.75 93.75) (end 159.25 92.25) (width 0.3) (layer F.Cu) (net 15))
 (segment (start 159.25 92.25) (end 159.25 86.09) (width 0.3) (layer F.Cu) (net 15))
 (segment (start 159.25 86.09) (end 159.59 85) (width 0.3) (layer F.Cu) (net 15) (status 20))
 (segment (start 145.75 71.75) (end 146.5 71.75) (width 0.3) (layer B.Cu) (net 7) (status 30))
 (segment (start 146.5 71.75) (end 153.75 80.75) (width 0.3) (layer B.Cu) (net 7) (status 10))
 (segment (start 153.75 80.75) (end 153.75 79) (width 0.3) (layer F.Cu) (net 7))
 (segment (start 157.79 74.96) (end 159.38 74.96) (width 0.3) (layer F.Cu) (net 7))
 (segment (start 153.75 79) (end 157.79 74.96) (width 0.3) (layer F.Cu) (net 7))
 (segment (start 167 74.96) (end 165.71 74.96) (width 0.3) (layer F.Cu) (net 12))
 (segment (start 160.15 67.65) (end 160.15 63.46) (width 0.3) (layer F.Cu) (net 12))
 (segment (start 162.5 70) (end 160.15 67.65) (width 0.3) (layer F.Cu) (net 12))
 (segment (start 162.5 71.75) (end 162.5 70) (width 0.3) (layer F.Cu) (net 12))
 (segment (start 165.71 74.96) (end 162.5 71.75) (width 0.3) (layer F.Cu) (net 12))
 (segment (start 137.16 70.485) (end 137.16 71.755) (width 2.7) (layer B.Cu) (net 5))
 (segment (start 137.16 71.755) (end 140.155 74.75) (width 2.7) (layer B.Cu) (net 5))
 (segment (start 140.155 74.75) (end 142.75 74.75) (width 2.7) (layer B.Cu) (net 5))
 (segment (start 142.75 74.75) (end 142.75 71.75) (width 0.3) (layer B.Cu) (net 5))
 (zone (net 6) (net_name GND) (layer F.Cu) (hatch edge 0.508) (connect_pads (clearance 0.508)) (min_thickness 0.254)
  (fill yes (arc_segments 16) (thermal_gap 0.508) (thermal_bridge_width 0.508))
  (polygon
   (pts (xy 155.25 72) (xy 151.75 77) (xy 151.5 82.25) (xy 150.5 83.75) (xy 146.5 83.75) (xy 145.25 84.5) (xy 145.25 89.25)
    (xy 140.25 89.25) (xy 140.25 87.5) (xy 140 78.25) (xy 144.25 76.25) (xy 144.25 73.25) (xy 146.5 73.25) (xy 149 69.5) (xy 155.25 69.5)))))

